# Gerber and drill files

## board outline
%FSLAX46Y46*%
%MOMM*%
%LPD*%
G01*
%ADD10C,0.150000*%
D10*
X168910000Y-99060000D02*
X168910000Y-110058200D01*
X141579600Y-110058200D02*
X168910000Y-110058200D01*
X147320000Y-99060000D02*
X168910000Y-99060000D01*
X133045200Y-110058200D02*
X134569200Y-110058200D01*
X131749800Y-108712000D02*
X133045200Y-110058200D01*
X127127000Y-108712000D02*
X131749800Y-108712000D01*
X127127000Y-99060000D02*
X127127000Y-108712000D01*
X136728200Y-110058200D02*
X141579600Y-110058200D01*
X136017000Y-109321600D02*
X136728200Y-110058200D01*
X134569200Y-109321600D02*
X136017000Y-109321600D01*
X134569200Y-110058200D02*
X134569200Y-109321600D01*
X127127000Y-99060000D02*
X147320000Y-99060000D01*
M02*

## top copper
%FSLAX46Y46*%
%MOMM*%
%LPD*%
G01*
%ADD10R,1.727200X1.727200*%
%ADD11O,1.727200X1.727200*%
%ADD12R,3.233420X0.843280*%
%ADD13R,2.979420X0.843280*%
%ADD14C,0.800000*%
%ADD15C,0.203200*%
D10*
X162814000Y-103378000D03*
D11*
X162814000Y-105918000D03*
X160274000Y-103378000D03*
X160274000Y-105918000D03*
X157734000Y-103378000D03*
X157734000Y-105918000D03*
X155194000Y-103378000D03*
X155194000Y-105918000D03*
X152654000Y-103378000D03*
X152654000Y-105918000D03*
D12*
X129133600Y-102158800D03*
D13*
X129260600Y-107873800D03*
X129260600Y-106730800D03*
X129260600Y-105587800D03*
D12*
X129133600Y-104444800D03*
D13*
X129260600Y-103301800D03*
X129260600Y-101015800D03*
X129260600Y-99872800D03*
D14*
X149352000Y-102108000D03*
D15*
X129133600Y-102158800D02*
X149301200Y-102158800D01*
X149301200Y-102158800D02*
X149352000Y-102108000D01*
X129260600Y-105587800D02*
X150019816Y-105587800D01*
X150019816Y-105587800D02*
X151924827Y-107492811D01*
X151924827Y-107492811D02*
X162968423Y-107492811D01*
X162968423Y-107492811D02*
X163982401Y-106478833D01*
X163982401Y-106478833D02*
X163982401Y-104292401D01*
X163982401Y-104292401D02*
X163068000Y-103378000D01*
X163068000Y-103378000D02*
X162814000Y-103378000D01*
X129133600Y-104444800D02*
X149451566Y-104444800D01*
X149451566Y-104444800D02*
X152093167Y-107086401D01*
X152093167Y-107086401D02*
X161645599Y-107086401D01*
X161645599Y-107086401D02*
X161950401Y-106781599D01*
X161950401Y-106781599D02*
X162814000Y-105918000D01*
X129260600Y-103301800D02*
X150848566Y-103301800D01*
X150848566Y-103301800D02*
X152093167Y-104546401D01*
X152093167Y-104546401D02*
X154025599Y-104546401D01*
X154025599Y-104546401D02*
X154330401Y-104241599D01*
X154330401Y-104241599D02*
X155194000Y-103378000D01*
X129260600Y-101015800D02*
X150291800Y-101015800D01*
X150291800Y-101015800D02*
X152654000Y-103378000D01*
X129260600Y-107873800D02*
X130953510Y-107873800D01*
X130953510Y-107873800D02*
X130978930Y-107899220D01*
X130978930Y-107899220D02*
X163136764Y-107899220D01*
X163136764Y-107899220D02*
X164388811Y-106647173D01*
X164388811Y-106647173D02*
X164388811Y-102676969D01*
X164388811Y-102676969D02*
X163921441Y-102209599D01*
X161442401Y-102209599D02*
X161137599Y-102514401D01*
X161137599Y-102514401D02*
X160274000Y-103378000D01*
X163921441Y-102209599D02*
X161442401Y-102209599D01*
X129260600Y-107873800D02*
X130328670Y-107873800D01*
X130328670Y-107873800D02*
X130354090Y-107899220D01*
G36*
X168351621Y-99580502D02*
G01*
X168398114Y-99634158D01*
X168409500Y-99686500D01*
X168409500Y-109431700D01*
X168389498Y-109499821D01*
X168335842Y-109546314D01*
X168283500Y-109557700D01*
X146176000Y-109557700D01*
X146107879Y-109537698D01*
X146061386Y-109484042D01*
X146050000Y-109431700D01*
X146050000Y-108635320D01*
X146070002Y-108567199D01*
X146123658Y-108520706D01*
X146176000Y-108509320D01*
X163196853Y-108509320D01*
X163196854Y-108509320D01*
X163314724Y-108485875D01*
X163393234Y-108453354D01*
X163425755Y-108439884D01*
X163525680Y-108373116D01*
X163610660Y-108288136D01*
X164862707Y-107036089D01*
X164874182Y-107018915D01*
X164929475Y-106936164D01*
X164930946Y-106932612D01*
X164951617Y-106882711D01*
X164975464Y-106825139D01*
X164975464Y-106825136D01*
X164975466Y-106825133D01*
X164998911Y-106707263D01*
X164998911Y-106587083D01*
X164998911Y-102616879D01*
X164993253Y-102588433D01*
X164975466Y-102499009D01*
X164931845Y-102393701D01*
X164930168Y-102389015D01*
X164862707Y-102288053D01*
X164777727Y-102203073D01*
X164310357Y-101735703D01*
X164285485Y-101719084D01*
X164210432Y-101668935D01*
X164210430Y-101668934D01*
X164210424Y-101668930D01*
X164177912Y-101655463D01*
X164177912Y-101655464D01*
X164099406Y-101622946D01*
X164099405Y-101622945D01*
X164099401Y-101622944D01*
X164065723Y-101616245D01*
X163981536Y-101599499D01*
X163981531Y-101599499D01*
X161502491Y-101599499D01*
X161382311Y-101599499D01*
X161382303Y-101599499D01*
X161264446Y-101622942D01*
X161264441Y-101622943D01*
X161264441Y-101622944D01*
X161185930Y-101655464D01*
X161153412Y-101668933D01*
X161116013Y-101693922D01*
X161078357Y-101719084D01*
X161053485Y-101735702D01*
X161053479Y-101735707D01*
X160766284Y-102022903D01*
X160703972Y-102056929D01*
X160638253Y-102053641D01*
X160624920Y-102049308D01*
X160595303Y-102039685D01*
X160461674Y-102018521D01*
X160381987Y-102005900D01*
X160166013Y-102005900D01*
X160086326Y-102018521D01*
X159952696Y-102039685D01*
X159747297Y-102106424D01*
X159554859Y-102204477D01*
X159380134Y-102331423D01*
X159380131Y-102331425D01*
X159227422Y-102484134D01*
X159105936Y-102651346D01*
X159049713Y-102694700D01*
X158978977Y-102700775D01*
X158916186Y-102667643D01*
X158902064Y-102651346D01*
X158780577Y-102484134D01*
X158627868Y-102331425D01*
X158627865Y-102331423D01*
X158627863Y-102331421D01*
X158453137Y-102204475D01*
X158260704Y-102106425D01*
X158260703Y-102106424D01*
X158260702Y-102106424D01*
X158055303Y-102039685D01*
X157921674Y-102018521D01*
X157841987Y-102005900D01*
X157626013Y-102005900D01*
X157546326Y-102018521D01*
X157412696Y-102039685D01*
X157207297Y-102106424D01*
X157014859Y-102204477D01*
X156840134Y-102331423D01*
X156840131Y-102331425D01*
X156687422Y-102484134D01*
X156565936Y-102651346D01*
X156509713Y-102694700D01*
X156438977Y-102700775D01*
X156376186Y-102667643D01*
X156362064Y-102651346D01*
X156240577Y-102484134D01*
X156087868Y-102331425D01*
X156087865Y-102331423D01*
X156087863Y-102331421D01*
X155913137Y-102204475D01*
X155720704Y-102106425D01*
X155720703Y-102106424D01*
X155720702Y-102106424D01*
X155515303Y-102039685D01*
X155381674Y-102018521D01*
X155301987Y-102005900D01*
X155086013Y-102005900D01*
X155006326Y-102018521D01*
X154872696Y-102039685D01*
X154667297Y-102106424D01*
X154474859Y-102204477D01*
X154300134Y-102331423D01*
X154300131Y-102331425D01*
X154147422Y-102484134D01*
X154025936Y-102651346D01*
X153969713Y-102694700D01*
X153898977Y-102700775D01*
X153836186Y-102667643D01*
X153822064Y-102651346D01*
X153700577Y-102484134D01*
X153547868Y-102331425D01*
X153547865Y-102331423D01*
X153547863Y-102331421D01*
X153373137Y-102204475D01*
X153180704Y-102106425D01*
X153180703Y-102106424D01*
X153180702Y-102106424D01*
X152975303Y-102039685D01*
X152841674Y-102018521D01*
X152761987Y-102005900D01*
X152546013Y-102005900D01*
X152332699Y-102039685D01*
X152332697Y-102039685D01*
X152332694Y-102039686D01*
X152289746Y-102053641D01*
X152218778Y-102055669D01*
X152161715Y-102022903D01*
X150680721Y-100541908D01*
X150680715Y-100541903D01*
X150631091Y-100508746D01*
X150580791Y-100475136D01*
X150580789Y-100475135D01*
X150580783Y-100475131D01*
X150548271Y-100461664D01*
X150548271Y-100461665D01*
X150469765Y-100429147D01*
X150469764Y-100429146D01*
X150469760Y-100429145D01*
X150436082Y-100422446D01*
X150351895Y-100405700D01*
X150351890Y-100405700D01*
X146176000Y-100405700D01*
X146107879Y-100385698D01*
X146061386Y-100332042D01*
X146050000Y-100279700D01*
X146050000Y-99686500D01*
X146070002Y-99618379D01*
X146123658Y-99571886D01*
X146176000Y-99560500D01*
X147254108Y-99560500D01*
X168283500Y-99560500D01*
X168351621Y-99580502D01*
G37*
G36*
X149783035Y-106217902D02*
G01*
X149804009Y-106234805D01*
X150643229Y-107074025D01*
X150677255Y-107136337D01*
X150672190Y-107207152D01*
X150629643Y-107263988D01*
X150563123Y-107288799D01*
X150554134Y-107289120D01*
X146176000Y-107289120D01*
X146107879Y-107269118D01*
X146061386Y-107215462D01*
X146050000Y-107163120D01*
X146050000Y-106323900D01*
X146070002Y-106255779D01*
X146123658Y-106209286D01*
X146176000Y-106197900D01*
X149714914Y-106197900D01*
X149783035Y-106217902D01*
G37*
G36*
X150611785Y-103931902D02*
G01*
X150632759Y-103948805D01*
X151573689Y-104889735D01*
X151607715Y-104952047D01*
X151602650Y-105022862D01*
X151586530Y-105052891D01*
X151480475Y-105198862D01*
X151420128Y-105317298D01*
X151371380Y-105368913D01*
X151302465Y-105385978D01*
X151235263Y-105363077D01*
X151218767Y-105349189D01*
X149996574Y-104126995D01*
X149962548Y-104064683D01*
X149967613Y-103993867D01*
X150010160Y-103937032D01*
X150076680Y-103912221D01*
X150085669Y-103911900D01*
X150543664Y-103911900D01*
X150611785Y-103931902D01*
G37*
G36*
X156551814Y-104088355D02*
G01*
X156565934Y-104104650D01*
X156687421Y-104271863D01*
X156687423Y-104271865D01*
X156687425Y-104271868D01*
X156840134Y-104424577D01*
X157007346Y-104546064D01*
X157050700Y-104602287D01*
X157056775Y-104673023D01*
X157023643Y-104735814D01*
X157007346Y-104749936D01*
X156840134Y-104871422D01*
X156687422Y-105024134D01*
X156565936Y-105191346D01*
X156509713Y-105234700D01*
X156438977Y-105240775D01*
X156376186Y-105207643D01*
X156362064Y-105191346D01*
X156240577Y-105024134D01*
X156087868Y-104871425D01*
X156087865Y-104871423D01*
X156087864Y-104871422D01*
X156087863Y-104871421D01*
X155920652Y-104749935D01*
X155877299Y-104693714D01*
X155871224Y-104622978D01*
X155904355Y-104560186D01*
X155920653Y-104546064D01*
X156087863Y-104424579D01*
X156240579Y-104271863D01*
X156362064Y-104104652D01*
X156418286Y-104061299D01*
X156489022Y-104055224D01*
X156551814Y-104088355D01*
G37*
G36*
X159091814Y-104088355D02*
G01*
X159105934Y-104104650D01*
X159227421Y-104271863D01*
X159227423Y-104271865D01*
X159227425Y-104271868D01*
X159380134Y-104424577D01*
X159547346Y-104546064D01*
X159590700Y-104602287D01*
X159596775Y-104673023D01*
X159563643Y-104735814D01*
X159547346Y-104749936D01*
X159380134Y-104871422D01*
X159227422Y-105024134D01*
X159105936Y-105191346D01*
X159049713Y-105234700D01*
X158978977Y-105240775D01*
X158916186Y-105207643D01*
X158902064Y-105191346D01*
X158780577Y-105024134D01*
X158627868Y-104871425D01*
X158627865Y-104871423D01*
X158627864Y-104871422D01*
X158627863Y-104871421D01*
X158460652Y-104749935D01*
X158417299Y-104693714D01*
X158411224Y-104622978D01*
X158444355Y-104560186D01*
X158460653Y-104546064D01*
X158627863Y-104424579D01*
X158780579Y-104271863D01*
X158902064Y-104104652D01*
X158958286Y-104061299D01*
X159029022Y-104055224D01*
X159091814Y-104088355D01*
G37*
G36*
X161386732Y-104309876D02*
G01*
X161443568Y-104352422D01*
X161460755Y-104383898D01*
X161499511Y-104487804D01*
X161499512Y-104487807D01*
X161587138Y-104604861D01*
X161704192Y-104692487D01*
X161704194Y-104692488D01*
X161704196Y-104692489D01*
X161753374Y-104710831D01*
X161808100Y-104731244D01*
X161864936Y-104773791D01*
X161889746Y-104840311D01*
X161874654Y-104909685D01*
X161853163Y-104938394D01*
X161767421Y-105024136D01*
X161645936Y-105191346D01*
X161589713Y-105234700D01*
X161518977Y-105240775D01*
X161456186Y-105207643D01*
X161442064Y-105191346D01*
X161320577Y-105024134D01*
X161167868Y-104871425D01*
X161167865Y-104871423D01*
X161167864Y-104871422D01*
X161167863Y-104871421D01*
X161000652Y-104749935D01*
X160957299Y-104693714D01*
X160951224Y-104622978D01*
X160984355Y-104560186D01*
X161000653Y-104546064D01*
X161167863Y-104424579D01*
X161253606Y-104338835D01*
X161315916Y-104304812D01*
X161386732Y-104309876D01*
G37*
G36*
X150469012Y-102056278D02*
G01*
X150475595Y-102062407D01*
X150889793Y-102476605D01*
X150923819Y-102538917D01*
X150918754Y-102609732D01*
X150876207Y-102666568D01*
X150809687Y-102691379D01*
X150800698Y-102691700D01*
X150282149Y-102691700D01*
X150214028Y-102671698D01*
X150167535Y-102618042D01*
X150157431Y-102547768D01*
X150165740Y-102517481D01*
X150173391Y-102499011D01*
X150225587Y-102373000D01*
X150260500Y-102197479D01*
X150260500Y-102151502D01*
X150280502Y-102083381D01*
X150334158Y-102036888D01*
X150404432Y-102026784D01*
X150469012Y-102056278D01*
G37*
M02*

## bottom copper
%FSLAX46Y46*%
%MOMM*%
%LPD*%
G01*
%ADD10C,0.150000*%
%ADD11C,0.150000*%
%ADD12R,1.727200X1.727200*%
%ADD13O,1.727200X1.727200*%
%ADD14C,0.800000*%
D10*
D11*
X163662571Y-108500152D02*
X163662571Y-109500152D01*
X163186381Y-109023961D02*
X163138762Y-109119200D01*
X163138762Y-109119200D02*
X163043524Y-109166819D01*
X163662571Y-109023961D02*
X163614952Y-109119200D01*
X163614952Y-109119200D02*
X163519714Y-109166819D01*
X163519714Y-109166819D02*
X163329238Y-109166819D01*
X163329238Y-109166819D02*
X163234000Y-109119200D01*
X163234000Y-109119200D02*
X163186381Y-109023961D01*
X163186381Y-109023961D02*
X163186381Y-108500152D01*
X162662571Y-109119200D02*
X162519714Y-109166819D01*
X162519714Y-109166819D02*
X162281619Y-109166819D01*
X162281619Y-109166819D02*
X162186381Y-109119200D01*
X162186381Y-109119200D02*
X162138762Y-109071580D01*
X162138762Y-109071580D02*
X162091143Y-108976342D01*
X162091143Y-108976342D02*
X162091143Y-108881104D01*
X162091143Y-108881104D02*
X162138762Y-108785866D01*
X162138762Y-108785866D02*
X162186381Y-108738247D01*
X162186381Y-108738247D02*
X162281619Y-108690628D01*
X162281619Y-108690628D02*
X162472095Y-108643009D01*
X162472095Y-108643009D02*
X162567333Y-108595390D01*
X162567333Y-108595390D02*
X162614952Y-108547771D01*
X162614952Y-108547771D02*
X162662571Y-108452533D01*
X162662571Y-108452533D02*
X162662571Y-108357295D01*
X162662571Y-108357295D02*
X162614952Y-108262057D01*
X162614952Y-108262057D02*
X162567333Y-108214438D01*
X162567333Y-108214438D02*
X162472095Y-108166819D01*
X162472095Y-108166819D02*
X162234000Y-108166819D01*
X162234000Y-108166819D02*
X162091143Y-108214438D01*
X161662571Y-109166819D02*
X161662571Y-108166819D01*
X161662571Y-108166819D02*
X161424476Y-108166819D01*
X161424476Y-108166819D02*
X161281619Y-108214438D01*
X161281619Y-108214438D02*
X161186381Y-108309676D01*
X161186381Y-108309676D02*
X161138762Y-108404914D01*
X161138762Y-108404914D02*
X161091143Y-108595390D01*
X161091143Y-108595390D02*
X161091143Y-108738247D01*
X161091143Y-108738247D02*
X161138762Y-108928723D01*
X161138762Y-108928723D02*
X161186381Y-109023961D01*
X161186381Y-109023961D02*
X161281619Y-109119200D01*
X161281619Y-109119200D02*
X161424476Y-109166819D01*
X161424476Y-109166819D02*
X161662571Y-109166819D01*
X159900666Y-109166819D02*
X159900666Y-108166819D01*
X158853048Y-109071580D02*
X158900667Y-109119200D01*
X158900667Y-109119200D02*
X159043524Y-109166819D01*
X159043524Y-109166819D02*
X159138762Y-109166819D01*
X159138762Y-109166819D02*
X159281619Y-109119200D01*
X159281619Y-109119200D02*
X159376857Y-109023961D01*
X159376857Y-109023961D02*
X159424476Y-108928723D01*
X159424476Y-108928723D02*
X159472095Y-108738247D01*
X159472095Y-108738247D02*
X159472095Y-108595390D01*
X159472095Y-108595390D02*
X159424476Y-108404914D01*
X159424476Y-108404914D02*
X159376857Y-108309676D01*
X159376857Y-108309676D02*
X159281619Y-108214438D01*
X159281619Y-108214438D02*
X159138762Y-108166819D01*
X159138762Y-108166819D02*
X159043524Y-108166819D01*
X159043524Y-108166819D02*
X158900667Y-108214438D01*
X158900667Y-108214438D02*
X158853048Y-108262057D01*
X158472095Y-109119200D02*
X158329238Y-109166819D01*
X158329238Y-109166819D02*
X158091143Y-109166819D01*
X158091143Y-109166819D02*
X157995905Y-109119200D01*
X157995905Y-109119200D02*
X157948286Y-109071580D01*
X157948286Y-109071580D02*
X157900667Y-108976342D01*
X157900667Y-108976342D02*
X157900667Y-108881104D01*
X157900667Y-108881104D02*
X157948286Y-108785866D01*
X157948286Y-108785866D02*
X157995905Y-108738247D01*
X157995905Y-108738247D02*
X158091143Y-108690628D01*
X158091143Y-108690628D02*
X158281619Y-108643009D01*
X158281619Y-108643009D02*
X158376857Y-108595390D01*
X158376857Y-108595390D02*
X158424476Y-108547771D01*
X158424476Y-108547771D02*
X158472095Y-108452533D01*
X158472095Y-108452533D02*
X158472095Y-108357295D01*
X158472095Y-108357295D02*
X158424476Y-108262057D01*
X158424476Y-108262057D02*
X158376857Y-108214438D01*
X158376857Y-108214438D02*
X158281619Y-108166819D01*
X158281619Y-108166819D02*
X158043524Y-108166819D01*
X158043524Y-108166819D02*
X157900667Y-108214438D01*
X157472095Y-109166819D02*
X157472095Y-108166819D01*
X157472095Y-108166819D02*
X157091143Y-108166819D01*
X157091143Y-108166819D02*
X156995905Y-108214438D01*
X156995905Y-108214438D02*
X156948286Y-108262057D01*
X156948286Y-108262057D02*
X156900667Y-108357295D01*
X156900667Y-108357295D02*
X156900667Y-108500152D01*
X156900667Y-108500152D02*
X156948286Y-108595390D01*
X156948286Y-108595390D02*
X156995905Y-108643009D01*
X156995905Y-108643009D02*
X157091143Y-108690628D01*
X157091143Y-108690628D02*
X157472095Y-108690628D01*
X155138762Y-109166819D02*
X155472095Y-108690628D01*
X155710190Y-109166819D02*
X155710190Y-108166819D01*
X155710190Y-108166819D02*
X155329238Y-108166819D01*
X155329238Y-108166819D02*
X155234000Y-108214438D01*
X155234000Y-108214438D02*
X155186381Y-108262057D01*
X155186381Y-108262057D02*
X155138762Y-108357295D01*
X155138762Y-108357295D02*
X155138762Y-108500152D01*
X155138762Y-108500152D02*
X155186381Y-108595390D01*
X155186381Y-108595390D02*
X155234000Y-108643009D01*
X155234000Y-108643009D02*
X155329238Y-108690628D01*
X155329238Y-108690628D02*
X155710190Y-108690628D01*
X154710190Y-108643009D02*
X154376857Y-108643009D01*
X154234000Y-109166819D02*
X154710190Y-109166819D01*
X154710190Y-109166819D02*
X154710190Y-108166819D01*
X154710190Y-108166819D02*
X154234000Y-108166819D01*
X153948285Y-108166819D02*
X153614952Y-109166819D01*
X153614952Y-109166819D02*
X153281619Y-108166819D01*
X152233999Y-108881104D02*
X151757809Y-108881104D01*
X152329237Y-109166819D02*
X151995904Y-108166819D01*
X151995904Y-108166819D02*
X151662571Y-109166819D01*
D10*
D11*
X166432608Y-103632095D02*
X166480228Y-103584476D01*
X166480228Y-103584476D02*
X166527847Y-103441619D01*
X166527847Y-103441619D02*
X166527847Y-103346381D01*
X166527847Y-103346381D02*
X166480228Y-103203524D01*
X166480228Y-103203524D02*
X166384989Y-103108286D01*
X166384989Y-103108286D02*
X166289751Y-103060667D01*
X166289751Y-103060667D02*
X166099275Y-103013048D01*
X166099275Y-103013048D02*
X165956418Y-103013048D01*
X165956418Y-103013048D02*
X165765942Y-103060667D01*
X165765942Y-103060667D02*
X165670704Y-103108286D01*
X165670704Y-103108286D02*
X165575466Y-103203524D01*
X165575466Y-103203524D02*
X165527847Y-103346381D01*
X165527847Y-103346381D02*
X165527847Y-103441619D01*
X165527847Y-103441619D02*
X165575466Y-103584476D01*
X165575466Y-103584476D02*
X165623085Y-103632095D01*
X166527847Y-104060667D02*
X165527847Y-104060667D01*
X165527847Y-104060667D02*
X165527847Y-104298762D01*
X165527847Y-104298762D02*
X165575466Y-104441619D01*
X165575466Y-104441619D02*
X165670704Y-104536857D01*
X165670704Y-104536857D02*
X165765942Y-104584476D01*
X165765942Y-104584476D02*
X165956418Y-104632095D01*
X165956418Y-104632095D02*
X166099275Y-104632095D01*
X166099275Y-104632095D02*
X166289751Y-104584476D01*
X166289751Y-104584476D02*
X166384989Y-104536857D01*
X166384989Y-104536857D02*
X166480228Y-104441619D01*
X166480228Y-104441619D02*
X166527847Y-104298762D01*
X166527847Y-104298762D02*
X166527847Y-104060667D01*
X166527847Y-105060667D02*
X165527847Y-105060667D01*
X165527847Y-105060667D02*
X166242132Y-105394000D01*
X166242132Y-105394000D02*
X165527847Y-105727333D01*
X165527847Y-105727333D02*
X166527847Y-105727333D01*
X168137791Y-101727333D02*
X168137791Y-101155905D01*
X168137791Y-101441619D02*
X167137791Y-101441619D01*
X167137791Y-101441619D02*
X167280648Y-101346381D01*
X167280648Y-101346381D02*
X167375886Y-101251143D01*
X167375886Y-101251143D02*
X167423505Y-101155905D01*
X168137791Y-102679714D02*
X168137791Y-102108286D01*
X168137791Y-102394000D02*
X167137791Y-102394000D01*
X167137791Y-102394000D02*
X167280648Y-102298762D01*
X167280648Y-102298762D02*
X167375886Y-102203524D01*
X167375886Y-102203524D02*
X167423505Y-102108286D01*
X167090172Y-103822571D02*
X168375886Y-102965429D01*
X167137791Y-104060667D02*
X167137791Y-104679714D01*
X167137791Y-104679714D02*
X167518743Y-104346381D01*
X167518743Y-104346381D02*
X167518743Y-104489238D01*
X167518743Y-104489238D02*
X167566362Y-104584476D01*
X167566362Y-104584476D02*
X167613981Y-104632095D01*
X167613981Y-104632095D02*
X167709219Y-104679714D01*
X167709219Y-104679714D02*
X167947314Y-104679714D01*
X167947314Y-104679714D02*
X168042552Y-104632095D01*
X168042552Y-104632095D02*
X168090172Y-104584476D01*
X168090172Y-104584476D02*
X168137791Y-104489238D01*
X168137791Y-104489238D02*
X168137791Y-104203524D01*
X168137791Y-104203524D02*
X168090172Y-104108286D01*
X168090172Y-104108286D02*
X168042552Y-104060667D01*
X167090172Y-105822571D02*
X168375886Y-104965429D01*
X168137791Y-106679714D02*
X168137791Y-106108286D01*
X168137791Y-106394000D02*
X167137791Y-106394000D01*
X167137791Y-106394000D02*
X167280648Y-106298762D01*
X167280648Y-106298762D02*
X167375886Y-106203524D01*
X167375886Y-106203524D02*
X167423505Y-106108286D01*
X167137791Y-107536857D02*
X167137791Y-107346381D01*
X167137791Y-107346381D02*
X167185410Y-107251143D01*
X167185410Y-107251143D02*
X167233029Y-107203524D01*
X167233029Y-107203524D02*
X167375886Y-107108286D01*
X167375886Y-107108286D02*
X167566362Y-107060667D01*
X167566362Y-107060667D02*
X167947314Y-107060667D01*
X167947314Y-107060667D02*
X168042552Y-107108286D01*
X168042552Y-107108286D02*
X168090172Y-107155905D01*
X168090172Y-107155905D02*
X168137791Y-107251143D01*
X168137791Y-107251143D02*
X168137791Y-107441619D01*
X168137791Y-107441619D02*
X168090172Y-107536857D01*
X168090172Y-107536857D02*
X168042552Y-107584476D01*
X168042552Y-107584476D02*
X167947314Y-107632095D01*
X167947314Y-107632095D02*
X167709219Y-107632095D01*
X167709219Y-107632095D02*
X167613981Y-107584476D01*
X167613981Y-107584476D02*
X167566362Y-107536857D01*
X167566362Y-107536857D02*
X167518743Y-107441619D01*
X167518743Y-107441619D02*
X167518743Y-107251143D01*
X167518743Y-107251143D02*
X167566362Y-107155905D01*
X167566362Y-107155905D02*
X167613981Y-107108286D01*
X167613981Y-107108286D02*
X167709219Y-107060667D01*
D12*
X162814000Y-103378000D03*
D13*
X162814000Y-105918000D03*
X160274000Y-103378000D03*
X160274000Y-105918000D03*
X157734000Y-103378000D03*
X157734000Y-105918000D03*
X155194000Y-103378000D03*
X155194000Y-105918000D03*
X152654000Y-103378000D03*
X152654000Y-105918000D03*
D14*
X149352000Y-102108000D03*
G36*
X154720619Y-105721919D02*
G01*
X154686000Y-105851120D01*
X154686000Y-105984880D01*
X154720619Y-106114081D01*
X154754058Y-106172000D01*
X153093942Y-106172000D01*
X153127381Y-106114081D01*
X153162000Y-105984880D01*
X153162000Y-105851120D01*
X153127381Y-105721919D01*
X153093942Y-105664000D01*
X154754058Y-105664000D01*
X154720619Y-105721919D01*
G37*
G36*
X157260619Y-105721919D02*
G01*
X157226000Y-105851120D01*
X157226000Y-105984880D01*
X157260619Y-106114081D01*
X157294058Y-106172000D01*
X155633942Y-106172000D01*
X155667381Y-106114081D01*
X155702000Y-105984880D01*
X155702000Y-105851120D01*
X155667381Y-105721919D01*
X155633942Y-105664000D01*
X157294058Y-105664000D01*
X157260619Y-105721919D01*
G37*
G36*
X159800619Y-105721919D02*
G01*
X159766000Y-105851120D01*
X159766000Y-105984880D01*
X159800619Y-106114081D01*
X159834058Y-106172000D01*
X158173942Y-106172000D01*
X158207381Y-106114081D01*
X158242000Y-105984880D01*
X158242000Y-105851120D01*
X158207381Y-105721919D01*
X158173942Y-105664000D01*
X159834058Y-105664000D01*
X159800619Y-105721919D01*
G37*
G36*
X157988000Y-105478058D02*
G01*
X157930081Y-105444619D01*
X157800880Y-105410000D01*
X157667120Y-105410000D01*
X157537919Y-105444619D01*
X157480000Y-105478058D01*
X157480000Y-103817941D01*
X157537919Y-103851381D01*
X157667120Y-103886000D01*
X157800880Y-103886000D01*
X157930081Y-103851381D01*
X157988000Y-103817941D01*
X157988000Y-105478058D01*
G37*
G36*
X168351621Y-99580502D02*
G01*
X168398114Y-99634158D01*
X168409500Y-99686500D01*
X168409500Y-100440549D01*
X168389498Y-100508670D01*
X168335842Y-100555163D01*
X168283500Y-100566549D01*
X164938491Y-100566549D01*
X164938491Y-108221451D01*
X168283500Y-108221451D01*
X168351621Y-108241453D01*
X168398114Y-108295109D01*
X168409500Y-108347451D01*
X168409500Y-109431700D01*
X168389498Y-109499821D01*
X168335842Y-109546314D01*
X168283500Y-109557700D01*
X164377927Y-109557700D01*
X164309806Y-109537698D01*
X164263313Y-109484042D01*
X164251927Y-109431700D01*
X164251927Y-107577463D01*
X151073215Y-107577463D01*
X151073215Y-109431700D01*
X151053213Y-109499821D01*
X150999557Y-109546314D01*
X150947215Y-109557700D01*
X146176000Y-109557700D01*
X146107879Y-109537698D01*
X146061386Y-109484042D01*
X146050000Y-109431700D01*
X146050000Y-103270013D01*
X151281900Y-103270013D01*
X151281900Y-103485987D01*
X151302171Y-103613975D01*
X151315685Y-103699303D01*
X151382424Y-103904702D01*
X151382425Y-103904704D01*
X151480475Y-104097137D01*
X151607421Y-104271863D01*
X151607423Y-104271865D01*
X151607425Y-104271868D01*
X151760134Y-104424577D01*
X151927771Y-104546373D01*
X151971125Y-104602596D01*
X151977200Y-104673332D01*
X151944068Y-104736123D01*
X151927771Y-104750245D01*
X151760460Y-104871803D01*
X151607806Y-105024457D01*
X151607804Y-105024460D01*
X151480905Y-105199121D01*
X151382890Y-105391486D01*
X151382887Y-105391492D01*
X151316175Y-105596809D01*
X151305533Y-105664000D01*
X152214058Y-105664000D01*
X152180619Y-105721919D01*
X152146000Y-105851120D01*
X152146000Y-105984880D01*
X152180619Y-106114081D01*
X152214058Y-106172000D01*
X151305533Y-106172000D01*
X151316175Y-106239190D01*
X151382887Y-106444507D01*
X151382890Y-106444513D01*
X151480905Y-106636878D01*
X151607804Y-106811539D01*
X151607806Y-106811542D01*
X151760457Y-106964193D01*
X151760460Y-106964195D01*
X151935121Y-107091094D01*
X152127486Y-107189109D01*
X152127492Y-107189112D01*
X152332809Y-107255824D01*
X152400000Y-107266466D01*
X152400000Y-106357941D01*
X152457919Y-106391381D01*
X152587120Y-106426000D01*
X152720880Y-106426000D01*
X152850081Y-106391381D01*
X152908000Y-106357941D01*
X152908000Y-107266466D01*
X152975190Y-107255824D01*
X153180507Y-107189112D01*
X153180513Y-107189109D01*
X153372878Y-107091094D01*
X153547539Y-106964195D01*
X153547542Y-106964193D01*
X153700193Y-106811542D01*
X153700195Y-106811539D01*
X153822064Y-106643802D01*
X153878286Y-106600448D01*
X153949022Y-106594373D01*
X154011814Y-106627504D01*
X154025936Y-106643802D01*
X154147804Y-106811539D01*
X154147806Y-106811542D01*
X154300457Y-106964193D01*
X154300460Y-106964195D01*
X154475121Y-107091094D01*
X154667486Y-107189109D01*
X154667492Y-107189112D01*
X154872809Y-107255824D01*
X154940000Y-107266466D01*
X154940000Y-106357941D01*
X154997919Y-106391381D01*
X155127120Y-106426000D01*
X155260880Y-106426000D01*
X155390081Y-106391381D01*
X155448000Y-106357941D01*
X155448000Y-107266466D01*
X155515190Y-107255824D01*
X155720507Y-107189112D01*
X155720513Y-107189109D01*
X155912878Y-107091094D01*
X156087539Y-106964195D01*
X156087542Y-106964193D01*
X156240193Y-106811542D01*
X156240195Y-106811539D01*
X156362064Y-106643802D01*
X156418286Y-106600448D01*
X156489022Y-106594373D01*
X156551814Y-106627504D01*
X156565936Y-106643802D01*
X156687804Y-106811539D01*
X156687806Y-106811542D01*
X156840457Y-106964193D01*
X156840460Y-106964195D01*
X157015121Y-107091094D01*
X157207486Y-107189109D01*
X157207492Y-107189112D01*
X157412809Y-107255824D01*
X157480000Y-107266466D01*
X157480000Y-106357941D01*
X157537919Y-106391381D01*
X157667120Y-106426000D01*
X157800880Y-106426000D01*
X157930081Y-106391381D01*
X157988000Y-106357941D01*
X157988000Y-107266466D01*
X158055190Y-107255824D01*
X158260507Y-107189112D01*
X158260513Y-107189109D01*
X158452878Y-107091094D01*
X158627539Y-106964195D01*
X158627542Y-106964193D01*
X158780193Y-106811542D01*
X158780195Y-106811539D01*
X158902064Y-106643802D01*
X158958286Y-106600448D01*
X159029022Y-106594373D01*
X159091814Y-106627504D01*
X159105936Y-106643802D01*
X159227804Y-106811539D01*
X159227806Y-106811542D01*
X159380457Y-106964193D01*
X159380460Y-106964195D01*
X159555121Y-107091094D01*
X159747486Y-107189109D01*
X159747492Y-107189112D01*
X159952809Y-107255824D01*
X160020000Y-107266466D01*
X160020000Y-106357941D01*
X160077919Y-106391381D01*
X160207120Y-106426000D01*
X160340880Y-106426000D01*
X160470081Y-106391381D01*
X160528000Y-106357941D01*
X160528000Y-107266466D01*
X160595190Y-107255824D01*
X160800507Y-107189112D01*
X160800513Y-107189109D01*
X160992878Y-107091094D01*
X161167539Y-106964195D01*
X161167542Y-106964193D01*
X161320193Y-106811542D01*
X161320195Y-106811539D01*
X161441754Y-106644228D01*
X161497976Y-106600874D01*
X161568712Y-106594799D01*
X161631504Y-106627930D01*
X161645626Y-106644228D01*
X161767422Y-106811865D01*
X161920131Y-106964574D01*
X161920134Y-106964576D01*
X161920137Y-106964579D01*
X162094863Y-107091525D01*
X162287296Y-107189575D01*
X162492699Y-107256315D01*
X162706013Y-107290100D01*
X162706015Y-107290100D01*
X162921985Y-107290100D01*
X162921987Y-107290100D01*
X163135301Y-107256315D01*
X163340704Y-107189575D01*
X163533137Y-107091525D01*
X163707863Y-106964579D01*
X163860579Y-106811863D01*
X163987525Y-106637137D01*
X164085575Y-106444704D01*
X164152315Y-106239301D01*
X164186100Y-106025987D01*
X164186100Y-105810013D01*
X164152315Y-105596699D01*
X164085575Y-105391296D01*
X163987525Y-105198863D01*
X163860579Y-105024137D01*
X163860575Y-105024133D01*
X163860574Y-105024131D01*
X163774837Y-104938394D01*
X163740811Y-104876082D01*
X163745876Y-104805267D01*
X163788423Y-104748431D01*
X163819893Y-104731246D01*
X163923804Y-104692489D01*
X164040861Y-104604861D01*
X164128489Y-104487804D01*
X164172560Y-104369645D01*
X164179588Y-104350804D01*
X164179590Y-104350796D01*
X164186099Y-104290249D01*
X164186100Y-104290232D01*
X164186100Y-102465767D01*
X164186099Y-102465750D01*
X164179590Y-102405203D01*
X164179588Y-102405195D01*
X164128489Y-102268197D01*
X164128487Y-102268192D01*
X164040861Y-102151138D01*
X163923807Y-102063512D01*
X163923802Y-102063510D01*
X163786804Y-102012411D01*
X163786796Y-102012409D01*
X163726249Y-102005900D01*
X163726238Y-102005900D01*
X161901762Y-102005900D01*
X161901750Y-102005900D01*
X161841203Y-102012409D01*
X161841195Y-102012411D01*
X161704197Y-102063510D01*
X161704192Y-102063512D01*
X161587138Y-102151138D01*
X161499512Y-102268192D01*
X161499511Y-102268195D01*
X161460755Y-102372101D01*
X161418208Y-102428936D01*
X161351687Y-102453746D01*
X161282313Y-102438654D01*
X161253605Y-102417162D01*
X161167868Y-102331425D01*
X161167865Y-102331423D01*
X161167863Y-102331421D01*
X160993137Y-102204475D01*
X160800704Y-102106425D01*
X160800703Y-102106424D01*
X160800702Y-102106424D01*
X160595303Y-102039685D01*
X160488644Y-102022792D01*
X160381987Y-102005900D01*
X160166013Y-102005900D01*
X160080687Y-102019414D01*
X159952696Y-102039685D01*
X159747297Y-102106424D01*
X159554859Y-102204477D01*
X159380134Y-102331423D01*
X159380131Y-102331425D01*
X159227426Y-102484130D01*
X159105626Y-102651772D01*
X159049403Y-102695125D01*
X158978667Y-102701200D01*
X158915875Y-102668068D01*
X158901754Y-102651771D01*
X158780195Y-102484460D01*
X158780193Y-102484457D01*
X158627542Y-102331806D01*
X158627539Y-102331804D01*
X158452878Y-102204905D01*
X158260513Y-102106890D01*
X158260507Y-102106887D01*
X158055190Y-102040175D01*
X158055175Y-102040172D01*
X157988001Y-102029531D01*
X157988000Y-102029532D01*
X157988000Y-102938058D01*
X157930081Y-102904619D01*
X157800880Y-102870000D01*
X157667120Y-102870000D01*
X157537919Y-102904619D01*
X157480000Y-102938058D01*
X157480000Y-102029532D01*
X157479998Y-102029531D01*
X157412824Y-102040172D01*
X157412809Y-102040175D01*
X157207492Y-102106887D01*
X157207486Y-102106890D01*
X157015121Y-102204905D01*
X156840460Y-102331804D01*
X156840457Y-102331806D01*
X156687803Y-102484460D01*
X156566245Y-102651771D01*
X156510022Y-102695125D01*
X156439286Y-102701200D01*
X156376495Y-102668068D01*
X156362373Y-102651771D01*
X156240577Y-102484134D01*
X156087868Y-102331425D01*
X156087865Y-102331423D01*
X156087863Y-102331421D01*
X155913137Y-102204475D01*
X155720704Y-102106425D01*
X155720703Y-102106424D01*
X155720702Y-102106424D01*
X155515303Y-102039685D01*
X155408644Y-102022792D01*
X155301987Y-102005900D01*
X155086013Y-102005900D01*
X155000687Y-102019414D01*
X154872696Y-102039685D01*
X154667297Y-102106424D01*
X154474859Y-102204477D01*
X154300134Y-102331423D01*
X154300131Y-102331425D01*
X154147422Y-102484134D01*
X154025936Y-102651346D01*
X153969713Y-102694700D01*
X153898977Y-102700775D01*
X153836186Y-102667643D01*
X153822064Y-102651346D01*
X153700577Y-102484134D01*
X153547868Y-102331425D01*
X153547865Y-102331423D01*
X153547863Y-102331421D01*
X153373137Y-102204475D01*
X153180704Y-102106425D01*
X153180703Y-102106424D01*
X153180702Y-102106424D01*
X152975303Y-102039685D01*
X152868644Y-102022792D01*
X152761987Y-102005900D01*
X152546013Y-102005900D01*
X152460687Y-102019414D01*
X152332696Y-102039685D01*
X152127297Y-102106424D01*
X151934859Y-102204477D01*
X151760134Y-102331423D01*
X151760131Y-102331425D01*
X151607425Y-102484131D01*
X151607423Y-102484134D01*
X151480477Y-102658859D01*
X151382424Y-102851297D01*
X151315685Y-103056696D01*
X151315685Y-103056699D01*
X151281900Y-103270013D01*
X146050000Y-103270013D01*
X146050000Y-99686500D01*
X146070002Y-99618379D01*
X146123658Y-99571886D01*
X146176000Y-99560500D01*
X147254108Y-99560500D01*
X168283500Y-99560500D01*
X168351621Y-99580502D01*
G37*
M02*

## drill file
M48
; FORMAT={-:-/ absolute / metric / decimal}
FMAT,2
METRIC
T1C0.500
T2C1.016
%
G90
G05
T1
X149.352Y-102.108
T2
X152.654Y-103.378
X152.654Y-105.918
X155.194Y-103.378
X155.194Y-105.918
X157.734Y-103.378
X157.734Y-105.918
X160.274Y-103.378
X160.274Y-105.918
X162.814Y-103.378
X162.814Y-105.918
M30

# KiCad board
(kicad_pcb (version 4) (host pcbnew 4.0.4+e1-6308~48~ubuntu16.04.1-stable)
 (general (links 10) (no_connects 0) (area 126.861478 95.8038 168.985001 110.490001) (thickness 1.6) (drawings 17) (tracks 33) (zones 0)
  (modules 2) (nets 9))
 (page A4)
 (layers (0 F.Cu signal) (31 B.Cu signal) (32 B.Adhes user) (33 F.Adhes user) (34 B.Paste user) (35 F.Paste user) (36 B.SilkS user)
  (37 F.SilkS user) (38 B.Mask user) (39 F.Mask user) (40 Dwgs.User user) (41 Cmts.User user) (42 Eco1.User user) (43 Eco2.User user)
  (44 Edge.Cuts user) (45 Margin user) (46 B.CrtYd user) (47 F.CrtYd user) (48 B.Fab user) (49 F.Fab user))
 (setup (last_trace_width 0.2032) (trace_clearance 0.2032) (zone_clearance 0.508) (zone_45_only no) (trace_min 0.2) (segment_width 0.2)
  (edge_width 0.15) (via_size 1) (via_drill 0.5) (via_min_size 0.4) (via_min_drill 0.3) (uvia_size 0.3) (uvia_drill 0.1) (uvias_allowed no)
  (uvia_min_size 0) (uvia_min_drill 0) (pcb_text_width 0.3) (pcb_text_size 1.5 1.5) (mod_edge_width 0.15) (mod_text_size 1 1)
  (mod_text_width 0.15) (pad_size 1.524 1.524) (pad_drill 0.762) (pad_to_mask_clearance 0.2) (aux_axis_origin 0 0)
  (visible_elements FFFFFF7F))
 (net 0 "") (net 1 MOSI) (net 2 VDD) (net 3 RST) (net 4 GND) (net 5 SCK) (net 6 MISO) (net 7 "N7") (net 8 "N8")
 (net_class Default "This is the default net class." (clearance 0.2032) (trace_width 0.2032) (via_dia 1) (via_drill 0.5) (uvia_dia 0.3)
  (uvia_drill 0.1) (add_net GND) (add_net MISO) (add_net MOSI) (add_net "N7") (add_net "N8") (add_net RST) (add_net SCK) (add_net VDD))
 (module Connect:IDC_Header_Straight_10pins (layer F.Cu) (at 162.814 103.378 180)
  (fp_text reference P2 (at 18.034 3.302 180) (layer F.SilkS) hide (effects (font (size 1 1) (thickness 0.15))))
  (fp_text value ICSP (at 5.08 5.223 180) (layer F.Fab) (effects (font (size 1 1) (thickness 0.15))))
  (pad 1 thru_hole rect (at 0 0 180) (size 1.7272 1.7272) (drill 1.016) (layers *.Cu *.Mask F.SilkS) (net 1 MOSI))
  (pad 2 thru_hole oval (at 0 -2.54 180) (size 1.7272 1.7272) (drill 1.016) (layers *.Cu *.Mask F.SilkS) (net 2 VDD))
  (pad 3 thru_hole oval (at 2.54 0 180) (size 1.7272 1.7272) (drill 1.016) (layers *.Cu *.Mask F.SilkS) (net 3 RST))
  (pad 4 thru_hole oval (at 2.54 -2.54 180) (size 1.7272 1.7272) (drill 1.016) (layers *.Cu *.Mask F.SilkS) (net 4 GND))
  (pad 5 thru_hole oval (at 5.08 0 180) (size 1.7272 1.7272) (drill 1.016) (layers *.Cu *.Mask F.SilkS) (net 4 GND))
  (pad 6 thru_hole oval (at 5.08 -2.54 180) (size 1.7272 1.7272) (drill 1.016) (layers *.Cu *.Mask F.SilkS) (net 4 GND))
  (pad 7 thru_hole oval (at 7.62 0 180) (size 1.7272 1.7272) (drill 1.016) (layers *.Cu *.Mask F.SilkS) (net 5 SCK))
  (pad 8 thru_hole oval (at 7.62 -2.54 180) (size 1.7272 1.7272) (drill 1.016) (layers *.Cu *.Mask F.SilkS) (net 4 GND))
  (pad 9 thru_hole oval (at 10.16 0 180) (size 1.7272 1.7272) (drill 1.016) (layers *.Cu *.Mask F.SilkS) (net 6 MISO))
  (pad 10 thru_hole oval (at 10.16 -2.54 180) (size 1.7272 1.7272) (drill 1.016) (layers *.Cu *.Mask F.SilkS) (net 4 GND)))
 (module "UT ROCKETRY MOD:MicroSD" (layer F.Cu) (at 134.874 97.282)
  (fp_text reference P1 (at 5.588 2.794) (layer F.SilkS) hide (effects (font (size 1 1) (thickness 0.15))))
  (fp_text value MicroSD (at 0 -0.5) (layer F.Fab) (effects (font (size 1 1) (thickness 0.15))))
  (pad 6 smd rect (at -5.7404 4.8768) (size 3.23342 0.84328) (layers F.Cu F.Paste F.Mask) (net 4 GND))
  (pad 1 smd rect (at -5.6134 10.5918) (size 2.97942 0.84328) (layers F.Cu F.Paste F.Mask) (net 3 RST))
  (pad 2 smd rect (at -5.6134 9.4488) (size 2.97942 0.84328) (layers F.Cu F.Paste F.Mask) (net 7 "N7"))
  (pad 3 smd rect (at -5.6134 8.3058) (size 2.97942 0.84328) (layers F.Cu F.Paste F.Mask) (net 1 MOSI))
  (pad 4 smd rect (at -5.7404 7.1628) (size 3.23342 0.84328) (layers F.Cu F.Paste F.Mask) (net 2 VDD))
  (pad 5 smd rect (at -5.6134 6.0198) (size 2.97942 0.84328) (layers F.Cu F.Paste F.Mask) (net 5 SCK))
  (pad 7 smd rect (at -5.6134 3.7338) (size 2.97942 0.84328) (layers F.Cu F.Paste F.Mask) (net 6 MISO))
  (pad 8 smd rect (at -5.6134 2.5908) (size 2.97942 0.84328) (layers F.Cu F.Paste F.Mask) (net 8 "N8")))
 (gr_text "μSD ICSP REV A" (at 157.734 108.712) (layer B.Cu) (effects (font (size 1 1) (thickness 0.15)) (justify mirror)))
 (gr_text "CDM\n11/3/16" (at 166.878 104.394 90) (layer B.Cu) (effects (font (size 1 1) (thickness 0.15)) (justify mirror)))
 (gr_line (start 168.91 99.06) (end 168.91 110.0582) (layer Edge.Cuts) (width 0.15))
 (gr_line (start 141.5796 110.0582) (end 168.91 110.0582) (layer Edge.Cuts) (width 0.15))
 (gr_line (start 147.32 99.06) (end 168.91 99.06) (layer Edge.Cuts) (width 0.15))
 (gr_line (start 133.0452 110.0582) (end 134.5692 110.0582) (layer Edge.Cuts) (width 0.15))
 (gr_line (start 131.7498 108.712) (end 133.0452 110.0582) (layer Edge.Cuts) (width 0.15))
 (gr_line (start 127.127 108.712) (end 131.7498 108.712) (layer Edge.Cuts) (width 0.15))
 (gr_line (start 127.127 99.06) (end 127.127 108.712) (layer Edge.Cuts) (width 0.15))
 (gr_line (start 136.7282 110.0582) (end 141.5796 110.0582) (layer Edge.Cuts) (width 0.15))
 (gr_line (start 136.017 109.3216) (end 136.7282 110.0582) (layer Edge.Cuts) (width 0.15))
 (gr_line (start 134.5692 109.3216) (end 136.017 109.3216) (layer Edge.Cuts) (width 0.15))
 (gr_line (start 134.5692 110.0582) (end 134.5692 109.3216) (layer Edge.Cuts) (width 0.15))
 (gr_line (start 127.127 99.06) (end 147.32 99.06) (layer Edge.Cuts) (width 0.15))
 (segment (start 129.1336 102.1588) (end 149.3012 102.1588) (width 0.2032) (layer F.Cu) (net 4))
 (segment (start 149.3012 102.1588) (end 149.352 102.108) (width 0.2032) (layer F.Cu) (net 4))
 (via (at 149.352 102.108) (size 0.8) (drill 0.5) (layers F.Cu B.Cu) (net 4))
 (segment (start 129.2606 105.5878) (end 150.019816 105.5878) (width 0.2032) (layer F.Cu) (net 1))
 (segment (start 150.019816 105.5878) (end 151.924827 107.492811) (width 0.2032) (layer F.Cu) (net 1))
 (segment (start 151.924827 107.492811) (end 162.968423 107.492811) (width 0.2032) (layer F.Cu) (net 1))
 (segment (start 162.968423 107.492811) (end 163.982401 106.478833) (width 0.2032) (layer F.Cu) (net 1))
 (segment (start 163.982401 106.478833) (end 163.982401 104.292401) (width 0.2032) (layer F.Cu) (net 1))
 (segment (start 163.982401 104.292401) (end 163.068 103.378) (width 0.2032) (layer F.Cu) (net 1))
 (segment (start 163.068 103.378) (end 162.814 103.378) (width 0.2032) (layer F.Cu) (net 1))
 (segment (start 129.1336 104.4448) (end 149.451566 104.4448) (width 0.2032) (layer F.Cu) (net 2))
 (segment (start 149.451566 104.4448) (end 152.093167 107.086401) (width 0.2032) (layer F.Cu) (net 2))
 (segment (start 152.093167 107.086401) (end 161.645599 107.086401) (width 0.2032) (layer F.Cu) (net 2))
 (segment (start 161.645599 107.086401) (end 161.950401 106.781599) (width 0.2032) (layer F.Cu) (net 2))
 (segment (start 161.950401 106.781599) (end 162.814 105.918) (width 0.2032) (layer F.Cu) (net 2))
 (segment (start 129.2606 103.3018) (end 150.848566 103.3018) (width 0.2032) (layer F.Cu) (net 5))
 (segment (start 150.848566 103.3018) (end 152.093167 104.546401) (width 0.2032) (layer F.Cu) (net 5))
 (segment (start 152.093167 104.546401) (end 154.025599 104.546401) (width 0.2032) (layer F.Cu) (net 5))
 (segment (start 154.025599 104.546401) (end 154.330401 104.241599) (width 0.2032) (layer F.Cu) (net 5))
 (segment (start 154.330401 104.241599) (end 155.194 103.378) (width 0.2032) (layer F.Cu) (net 5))
 (segment (start 129.2606 101.0158) (end 150.2918 101.0158) (width 0.2032) (layer F.Cu) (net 6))
 (segment (start 150.2918 101.0158) (end 152.654 103.378) (width 0.2032) (layer F.Cu) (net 6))
 (segment (start 129.2606 107.8738) (end 130.95351 107.8738) (width 0.2032) (layer F.Cu) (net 3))
 (segment (start 130.95351 107.8738) (end 130.97893 107.89922) (width 0.2032) (layer F.Cu) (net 3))
 (segment (start 130.97893 107.89922) (end 163.136764 107.89922) (width 0.2032) (layer F.Cu) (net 3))
 (segment (start 163.136764 107.89922) (end 164.388811 106.647173) (width 0.2032) (layer F.Cu) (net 3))
 (segment (start 164.388811 106.647173) (end 164.388811 102.676969) (width 0.2032) (layer F.Cu) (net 3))
 (segment (start 164.388811 102.676969) (end 163.921441 102.209599) (width 0.2032) (layer F.Cu) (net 3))
 (segment (start 161.442401 102.209599) (end 161.137599 102.514401) (width 0.2032) (layer F.Cu) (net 3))
 (segment (start 161.137599 102.514401) (end 160.274 103.378) (width 0.2032) (layer F.Cu) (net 3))
 (segment (start 163.921441 102.209599) (end 161.442401 102.209599) (width 0.2032) (layer F.Cu) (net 3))
 (segment (start 129.2606 107.8738) (end 130.32867 107.8738) (width 0.2032) (layer F.Cu) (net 3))
 (segment (start 130.32867 107.8738) (end 130.35409 107.89922) (width 0.2032) (layer F.Cu) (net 3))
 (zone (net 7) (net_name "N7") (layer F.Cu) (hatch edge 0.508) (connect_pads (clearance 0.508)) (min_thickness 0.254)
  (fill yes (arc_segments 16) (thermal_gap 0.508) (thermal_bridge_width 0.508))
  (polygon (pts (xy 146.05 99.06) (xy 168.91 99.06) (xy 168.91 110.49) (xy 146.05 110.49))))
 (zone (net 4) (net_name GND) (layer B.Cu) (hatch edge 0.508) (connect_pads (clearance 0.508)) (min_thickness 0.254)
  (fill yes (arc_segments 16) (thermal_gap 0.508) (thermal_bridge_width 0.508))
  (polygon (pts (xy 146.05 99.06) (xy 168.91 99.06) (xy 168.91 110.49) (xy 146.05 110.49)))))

